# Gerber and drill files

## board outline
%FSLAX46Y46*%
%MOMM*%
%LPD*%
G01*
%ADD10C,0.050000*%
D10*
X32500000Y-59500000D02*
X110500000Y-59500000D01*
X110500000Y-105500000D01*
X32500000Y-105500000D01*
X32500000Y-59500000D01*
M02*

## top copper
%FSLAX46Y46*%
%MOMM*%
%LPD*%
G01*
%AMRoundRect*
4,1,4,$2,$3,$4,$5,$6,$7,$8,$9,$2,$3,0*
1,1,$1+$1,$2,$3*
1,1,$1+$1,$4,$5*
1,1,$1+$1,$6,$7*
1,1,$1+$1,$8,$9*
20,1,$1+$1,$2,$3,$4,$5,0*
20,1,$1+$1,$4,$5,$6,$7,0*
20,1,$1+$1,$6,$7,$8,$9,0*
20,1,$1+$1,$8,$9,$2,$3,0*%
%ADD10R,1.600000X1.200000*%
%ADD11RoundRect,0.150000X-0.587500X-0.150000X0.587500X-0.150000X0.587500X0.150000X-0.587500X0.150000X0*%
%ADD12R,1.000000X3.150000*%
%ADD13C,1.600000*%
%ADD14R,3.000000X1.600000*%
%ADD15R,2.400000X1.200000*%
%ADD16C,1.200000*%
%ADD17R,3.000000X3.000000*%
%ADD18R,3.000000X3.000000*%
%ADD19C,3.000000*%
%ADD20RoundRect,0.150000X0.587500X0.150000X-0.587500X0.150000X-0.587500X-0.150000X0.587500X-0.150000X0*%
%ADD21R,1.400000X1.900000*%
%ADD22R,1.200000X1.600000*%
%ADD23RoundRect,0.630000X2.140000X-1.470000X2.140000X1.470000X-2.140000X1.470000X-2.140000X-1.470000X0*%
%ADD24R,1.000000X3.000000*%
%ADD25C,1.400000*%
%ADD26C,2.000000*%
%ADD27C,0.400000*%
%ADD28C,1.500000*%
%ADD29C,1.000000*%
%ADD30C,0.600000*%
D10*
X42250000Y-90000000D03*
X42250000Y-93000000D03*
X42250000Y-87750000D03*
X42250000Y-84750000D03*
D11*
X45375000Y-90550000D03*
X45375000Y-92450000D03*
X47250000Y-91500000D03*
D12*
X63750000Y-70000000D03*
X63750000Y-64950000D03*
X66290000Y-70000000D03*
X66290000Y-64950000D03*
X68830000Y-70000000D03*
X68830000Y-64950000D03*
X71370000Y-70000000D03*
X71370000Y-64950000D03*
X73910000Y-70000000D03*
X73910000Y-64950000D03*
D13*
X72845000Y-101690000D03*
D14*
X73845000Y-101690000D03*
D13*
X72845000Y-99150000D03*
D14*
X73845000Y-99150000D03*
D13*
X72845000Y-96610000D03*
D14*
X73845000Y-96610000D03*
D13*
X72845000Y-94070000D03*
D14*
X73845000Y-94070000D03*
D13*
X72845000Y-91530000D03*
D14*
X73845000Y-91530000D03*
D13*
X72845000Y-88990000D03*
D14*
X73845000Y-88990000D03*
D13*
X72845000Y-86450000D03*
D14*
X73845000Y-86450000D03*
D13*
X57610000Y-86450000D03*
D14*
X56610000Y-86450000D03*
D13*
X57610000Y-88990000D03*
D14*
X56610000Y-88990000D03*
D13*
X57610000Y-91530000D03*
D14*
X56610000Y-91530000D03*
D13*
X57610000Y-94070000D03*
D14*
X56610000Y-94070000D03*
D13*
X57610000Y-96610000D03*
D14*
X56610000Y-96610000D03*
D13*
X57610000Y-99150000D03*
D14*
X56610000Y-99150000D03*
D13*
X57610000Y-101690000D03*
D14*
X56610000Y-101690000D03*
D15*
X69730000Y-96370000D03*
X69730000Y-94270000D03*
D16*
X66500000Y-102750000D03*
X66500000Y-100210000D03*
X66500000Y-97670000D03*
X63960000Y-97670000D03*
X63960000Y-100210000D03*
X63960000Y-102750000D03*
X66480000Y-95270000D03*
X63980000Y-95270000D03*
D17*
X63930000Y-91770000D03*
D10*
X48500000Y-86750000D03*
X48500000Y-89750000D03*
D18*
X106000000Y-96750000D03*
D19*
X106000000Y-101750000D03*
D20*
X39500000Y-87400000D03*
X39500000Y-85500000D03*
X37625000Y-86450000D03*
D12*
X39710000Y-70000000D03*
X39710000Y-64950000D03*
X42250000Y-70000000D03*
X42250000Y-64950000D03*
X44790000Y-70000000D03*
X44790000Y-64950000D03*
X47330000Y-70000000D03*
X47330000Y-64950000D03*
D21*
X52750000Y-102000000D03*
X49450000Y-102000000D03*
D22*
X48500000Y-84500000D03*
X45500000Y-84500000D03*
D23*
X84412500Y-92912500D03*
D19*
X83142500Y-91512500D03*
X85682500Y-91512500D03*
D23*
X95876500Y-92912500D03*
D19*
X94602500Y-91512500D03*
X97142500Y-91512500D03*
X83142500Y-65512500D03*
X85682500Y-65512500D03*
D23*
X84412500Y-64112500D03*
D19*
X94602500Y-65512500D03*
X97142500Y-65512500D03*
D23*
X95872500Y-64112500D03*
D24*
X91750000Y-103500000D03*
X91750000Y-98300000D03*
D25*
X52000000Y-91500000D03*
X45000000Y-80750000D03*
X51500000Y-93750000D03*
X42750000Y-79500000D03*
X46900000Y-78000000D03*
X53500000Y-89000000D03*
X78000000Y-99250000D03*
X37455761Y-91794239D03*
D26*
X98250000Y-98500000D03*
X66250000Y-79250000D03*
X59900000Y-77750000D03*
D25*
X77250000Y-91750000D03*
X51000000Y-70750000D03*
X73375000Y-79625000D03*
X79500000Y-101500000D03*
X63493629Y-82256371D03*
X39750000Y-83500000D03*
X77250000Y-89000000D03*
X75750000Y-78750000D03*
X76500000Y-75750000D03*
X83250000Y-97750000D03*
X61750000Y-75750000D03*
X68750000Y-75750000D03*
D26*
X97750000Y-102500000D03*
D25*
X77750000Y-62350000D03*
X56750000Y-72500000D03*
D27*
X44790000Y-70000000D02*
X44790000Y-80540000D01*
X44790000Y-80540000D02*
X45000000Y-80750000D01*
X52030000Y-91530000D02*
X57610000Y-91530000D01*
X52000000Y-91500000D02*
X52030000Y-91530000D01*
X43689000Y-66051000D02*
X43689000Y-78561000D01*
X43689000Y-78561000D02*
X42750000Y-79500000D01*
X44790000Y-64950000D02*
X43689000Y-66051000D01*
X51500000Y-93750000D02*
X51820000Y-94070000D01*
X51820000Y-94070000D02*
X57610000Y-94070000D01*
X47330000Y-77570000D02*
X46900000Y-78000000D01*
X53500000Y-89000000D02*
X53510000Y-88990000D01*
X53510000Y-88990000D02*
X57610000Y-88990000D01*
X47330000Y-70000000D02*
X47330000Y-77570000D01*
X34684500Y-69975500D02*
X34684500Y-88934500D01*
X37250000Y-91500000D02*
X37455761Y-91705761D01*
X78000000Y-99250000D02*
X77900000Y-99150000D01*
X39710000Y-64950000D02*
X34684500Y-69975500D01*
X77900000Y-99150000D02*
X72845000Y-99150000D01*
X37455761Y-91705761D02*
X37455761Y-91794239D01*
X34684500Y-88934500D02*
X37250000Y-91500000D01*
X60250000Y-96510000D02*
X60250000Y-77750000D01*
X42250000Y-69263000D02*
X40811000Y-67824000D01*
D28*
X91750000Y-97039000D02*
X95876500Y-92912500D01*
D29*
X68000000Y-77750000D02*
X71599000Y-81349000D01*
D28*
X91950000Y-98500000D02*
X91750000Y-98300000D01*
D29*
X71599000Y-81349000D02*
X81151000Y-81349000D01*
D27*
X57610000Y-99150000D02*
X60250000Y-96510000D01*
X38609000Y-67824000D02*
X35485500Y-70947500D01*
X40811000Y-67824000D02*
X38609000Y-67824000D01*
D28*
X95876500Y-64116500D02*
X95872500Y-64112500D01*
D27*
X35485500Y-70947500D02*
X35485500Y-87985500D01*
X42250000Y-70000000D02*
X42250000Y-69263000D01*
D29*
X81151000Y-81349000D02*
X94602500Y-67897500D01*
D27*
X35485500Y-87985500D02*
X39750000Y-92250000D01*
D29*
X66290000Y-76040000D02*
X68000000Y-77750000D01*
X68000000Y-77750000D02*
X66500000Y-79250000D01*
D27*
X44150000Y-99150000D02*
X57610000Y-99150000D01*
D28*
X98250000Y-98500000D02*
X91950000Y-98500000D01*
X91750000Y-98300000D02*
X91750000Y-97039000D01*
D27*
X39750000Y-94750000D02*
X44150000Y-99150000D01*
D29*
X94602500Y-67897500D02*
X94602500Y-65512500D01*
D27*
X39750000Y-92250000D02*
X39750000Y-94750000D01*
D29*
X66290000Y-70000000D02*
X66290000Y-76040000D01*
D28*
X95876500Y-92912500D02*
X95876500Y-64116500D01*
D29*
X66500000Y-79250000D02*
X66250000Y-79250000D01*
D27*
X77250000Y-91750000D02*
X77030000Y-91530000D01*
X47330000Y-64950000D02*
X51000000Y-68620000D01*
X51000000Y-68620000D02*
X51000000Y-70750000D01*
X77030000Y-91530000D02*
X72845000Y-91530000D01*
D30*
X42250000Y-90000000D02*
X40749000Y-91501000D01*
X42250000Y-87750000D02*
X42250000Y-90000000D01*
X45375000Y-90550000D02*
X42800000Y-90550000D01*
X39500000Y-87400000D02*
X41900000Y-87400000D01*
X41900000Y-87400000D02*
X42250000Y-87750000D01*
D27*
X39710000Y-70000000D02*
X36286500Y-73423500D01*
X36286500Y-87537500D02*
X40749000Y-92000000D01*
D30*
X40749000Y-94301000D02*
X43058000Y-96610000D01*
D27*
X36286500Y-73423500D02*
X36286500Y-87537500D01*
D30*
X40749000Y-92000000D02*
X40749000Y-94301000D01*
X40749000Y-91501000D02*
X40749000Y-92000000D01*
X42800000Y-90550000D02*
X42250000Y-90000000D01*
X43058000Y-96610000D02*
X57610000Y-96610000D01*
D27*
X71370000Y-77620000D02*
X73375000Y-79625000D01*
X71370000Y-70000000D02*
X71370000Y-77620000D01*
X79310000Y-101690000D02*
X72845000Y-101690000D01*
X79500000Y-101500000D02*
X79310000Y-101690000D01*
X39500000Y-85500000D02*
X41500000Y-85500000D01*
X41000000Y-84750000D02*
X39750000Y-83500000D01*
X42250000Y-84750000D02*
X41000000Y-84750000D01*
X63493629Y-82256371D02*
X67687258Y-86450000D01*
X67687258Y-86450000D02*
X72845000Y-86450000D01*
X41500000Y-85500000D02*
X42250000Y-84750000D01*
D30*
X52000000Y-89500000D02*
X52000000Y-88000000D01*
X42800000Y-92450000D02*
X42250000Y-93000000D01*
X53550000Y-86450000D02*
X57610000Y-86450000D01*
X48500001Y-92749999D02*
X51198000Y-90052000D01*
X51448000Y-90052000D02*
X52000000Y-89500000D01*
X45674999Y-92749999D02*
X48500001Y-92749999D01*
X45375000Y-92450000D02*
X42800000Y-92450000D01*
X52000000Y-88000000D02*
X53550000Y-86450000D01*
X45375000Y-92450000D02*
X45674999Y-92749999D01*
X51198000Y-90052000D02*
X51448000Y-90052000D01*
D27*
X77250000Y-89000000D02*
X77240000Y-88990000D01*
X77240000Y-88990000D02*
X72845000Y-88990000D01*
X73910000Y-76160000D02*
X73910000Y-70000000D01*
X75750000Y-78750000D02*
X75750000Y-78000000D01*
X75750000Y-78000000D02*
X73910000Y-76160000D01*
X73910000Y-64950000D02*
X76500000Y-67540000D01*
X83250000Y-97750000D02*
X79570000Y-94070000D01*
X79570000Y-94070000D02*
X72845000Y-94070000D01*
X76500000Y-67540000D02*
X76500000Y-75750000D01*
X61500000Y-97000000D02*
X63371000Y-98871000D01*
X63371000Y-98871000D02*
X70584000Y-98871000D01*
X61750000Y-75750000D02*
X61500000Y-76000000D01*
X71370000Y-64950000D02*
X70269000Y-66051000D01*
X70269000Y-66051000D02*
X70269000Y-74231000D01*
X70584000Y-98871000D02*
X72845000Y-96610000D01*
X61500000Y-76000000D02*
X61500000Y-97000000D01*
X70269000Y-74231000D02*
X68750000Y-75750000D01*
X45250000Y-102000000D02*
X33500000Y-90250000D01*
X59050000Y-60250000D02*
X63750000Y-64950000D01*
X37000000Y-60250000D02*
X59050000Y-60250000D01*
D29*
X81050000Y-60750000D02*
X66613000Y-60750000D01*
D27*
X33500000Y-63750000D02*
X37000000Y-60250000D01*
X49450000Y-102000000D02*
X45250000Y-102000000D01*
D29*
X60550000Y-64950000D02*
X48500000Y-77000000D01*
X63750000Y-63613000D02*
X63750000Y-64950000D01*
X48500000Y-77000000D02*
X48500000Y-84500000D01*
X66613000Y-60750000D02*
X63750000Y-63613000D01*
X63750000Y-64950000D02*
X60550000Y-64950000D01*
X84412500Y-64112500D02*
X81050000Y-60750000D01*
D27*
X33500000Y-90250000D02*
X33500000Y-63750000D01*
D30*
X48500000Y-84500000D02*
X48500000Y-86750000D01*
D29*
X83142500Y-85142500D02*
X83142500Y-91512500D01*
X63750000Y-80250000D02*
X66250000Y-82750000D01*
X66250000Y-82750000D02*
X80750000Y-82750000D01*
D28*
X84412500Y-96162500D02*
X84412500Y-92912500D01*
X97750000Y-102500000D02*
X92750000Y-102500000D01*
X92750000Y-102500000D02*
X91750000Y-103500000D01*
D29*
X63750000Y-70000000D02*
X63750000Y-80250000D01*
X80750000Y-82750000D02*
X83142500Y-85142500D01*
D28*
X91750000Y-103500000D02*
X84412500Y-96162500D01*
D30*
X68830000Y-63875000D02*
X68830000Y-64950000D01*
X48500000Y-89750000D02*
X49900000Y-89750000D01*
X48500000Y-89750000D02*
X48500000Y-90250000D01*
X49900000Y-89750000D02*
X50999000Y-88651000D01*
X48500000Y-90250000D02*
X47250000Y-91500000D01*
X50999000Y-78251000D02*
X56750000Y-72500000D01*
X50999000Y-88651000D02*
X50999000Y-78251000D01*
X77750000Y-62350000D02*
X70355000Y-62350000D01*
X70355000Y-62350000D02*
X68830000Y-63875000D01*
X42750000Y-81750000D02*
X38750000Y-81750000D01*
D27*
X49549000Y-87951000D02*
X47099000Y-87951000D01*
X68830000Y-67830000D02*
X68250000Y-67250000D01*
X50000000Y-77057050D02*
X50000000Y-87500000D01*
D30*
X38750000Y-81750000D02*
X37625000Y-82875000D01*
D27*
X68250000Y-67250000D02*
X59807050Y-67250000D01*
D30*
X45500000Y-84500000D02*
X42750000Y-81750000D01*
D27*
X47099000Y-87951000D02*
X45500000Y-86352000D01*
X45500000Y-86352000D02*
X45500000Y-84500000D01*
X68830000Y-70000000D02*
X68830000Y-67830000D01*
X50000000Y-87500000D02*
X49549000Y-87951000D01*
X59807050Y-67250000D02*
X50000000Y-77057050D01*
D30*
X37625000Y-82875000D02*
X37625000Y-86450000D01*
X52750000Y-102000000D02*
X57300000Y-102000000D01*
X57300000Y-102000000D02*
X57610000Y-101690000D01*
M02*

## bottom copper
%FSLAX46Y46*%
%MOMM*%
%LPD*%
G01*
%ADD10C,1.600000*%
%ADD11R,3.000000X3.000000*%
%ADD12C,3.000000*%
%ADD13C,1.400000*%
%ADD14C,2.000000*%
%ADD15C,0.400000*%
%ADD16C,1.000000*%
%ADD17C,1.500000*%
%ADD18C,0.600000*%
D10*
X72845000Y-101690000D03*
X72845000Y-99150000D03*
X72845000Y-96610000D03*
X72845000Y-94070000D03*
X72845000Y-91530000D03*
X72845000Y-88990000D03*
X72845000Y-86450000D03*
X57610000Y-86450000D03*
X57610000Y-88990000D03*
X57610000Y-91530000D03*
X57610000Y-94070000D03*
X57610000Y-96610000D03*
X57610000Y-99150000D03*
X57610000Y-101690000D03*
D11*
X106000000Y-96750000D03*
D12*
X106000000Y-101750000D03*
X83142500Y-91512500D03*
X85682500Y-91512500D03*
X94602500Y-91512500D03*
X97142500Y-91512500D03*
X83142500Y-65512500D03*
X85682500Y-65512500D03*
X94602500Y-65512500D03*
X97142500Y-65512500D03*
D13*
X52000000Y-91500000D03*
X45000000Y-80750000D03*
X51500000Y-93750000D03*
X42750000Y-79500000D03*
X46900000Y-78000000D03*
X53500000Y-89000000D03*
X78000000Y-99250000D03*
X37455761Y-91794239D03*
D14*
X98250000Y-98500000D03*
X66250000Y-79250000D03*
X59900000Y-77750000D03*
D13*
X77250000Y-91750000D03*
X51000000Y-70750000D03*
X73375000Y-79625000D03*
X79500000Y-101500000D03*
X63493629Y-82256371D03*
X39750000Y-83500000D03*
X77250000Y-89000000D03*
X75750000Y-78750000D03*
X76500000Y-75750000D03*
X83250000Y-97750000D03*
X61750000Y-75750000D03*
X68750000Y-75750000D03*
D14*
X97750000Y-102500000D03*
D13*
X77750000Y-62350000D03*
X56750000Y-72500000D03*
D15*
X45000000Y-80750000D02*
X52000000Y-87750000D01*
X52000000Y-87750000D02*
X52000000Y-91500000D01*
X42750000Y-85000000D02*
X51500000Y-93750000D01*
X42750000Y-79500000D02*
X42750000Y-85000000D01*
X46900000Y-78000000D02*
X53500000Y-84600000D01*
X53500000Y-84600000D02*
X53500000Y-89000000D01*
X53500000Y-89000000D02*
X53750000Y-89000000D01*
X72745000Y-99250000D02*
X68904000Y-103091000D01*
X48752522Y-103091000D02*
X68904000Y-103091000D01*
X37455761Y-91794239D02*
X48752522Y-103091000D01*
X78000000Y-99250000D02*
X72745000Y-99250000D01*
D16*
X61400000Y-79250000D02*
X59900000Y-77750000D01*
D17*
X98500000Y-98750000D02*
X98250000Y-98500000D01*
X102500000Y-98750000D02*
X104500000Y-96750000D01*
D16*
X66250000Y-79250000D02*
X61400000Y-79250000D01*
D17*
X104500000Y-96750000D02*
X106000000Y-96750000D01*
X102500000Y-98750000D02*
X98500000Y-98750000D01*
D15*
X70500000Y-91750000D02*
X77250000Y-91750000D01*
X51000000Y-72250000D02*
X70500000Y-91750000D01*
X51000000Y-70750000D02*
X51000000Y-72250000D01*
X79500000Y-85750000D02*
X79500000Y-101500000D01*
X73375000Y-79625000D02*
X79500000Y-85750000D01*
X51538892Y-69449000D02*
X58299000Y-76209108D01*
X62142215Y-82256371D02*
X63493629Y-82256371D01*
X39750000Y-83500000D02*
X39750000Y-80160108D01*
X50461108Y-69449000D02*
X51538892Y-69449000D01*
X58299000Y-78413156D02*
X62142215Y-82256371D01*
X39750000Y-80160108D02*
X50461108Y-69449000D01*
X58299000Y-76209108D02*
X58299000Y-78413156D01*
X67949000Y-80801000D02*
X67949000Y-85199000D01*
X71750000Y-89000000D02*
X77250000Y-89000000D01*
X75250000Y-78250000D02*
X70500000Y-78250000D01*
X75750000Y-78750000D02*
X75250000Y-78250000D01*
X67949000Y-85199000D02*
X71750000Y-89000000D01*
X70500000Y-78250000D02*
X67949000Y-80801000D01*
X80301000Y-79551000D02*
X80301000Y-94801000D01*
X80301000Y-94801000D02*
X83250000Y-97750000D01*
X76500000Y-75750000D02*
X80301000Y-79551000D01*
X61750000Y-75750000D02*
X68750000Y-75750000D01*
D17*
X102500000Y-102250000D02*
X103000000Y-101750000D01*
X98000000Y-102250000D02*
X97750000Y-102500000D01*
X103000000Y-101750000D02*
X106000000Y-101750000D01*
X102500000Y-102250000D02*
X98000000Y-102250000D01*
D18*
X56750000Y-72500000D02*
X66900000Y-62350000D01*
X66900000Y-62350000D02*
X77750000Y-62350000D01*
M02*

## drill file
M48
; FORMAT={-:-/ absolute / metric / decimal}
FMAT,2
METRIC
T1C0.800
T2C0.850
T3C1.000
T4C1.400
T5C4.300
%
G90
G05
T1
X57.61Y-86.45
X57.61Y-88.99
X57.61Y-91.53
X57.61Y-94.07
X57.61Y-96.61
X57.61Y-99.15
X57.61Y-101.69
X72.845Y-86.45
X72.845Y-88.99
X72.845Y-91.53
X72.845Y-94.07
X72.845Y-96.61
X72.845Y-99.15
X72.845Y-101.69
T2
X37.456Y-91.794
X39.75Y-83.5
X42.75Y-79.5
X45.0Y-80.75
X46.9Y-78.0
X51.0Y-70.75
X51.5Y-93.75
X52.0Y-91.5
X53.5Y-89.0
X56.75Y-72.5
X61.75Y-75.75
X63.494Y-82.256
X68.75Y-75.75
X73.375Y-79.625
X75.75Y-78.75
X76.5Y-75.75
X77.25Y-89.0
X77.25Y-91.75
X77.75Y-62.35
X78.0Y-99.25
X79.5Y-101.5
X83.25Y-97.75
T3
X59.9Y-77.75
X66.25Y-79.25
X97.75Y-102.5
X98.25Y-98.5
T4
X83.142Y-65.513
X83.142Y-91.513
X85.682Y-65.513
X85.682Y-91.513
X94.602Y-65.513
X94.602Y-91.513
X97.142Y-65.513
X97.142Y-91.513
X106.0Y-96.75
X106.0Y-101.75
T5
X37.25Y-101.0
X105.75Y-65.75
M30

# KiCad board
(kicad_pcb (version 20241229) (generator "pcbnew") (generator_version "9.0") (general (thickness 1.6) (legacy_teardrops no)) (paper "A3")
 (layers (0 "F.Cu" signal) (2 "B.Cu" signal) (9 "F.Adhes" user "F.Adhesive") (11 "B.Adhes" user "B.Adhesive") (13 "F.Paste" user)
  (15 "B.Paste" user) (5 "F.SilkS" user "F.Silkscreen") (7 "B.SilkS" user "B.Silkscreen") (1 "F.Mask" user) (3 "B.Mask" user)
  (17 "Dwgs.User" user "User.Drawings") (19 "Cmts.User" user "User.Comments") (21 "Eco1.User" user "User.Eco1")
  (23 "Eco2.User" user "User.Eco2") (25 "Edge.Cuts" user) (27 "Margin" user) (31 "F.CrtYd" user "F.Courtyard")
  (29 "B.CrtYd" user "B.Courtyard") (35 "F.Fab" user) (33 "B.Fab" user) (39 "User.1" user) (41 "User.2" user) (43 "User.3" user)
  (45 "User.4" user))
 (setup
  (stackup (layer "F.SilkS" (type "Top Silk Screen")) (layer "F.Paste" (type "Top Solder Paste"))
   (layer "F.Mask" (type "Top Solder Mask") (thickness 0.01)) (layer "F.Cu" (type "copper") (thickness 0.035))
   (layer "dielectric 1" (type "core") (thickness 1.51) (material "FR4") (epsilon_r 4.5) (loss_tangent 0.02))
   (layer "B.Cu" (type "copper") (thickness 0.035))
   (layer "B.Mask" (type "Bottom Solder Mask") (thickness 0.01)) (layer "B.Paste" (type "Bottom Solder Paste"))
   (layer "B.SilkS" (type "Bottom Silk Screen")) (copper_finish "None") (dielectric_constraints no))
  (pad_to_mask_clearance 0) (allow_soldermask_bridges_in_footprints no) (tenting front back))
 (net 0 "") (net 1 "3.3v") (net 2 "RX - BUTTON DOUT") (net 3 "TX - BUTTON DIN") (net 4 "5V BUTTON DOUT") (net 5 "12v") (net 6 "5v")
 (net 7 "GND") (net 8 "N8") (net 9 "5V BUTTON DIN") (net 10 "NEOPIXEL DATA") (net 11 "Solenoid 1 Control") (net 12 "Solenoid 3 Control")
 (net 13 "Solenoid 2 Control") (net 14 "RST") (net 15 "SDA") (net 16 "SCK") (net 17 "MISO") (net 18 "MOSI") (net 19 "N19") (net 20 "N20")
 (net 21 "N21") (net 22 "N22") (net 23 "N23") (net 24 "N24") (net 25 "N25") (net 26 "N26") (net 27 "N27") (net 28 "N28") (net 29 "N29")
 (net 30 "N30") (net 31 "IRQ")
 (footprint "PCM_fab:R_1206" (layer "F.Cu") (at 42.25 91.5 -90)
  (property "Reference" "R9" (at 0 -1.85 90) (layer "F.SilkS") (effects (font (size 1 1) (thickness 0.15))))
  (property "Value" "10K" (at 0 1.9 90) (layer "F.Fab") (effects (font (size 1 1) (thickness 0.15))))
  (pad "1" smd rect (at -1.5 0 270) (size 1.2 1.6) (layers "F.Cu" "F.Mask" "F.Paste") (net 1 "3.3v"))
  (pad "2" smd rect (at 1.5 0 270) (size 1.2 1.6) (layers "F.Cu" "F.Mask" "F.Paste") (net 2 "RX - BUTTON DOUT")))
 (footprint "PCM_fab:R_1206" (layer "F.Cu") (at 42.25 86.25 90)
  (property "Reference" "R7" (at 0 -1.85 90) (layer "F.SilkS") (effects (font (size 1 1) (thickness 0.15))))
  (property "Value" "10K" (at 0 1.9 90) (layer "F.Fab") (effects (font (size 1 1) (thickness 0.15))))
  (pad "1" smd rect (at -1.5 0 90) (size 1.2 1.6) (layers "F.Cu" "F.Mask" "F.Paste") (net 1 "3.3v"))
  (pad "2" smd rect (at 1.5 0 90) (size 1.2 1.6) (layers "F.Cu" "F.Mask" "F.Paste") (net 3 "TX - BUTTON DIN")))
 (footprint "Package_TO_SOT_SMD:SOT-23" (layer "F.Cu") (at 46.3125 91.5)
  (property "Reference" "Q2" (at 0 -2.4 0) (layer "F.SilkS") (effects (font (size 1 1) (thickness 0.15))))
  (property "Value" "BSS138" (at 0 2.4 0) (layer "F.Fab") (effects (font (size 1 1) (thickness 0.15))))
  (pad "1" smd roundrect (at -0.9375 -0.95) (size 1.475 0.6) (layers "F.Cu" "F.Mask" "F.Paste") (roundrect_rratio 0.25) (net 1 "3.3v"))
  (pad "2" smd roundrect (at -0.9375 0.95) (size 1.475 0.6) (layers "F.Cu" "F.Mask" "F.Paste") (roundrect_rratio 0.25)
   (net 2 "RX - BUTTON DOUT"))
  (pad "3" smd roundrect (at 0.9375 0) (size 1.475 0.6) (layers "F.Cu" "F.Mask" "F.Paste") (roundrect_rratio 0.25) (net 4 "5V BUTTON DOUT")))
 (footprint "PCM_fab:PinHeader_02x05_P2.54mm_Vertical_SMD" (layer "F.Cu") (at 68.83 67.475 90)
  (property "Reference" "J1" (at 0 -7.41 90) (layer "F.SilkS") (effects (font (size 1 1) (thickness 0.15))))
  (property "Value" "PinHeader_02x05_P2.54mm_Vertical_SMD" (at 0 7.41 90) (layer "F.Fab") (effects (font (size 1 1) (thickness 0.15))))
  (pad "1" smd rect (at -2.525 -5.08 90) (size 3.15 1) (layers "F.Cu" "F.Mask" "F.Paste") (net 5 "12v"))
  (pad "2" smd rect (at 2.525 -5.08 90) (size 3.15 1) (layers "F.Cu" "F.Mask" "F.Paste") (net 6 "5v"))
  (pad "3" smd rect (at -2.525 -2.54 90) (size 3.15 1) (layers "F.Cu" "F.Mask" "F.Paste") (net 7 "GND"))
  (pad "4" smd rect (at 2.525 -2.54 90) (size 3.15 1) (layers "F.Cu" "F.Mask" "F.Paste") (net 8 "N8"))
  (pad "5" smd rect (at -2.525 0 90) (size 3.15 1) (layers "F.Cu" "F.Mask" "F.Paste") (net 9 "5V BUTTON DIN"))
  (pad "6" smd rect (at 2.525 0 90) (size 3.15 1) (layers "F.Cu" "F.Mask" "F.Paste") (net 4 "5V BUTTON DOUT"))
  (pad "7" smd rect (at -2.525 2.54 90) (size 3.15 1) (layers "F.Cu" "F.Mask" "F.Paste") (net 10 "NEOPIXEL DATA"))
  (pad "8" smd rect (at 2.525 2.54 90) (size 3.15 1) (layers "F.Cu" "F.Mask" "F.Paste") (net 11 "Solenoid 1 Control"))
  (pad "9" smd rect (at -2.525 5.08 90) (size 3.15 1) (layers "F.Cu" "F.Mask" "F.Paste") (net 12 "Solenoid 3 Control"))
  (pad "10" smd rect (at 2.525 5.08 90) (size 3.15 1) (layers "F.Cu" "F.Mask" "F.Paste") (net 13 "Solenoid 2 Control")))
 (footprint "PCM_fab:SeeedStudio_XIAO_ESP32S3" (layer "F.Cu") (at 65.23 94.07 180)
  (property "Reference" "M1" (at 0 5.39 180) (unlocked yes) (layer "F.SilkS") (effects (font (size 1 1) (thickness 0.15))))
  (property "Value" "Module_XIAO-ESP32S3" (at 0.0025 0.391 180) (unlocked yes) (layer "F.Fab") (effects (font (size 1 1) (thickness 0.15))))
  (pad "1" thru_hole circle (at -7.615 -7.62 180) (size 1.6 1.6) (drill 0.8) (layers "*.Cu" "*.Mask") (remove_unused_layers no)
   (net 10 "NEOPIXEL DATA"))
  (pad "1" smd rect (at -7.615 -7.62 180) (size 3 1.6) (drill (offset -1 0)) (layers "F.Cu" "F.Mask" "F.Paste") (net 10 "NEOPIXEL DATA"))
  (pad "2" thru_hole circle (at -7.615 -5.08 180) (size 1.6 1.6) (drill 0.8) (layers "*.Cu" "*.Mask") (remove_unused_layers no)
   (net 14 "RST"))
  (pad "2" smd rect (at -7.615 -5.08 180) (size 3 1.6) (drill (offset -1 0)) (layers "F.Cu" "F.Mask" "F.Paste") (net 14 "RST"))
  (pad "3" thru_hole circle (at -7.615 -2.54 180) (size 1.6 1.6) (drill 0.8) (layers "*.Cu" "*.Mask") (remove_unused_layers no)
   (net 11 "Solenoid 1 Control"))
  (pad "3" smd rect (at -7.615 -2.54 180) (size 3 1.6) (drill (offset -1 0)) (layers "F.Cu" "F.Mask" "F.Paste")
   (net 11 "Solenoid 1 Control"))
  (pad "4" thru_hole circle (at -7.615 0 180) (size 1.6 1.6) (drill 0.8) (layers "*.Cu" "*.Mask") (remove_unused_layers no)
   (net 13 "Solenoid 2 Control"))
  (pad "4" smd rect (at -7.615 0 180) (size 3 1.6) (drill (offset -1 0)) (layers "F.Cu" "F.Mask" "F.Paste") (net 13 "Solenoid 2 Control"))
  (pad "5" thru_hole circle (at -7.615 2.54 180) (size 1.6 1.6) (drill 0.8) (layers "*.Cu" "*.Mask") (remove_unused_layers no)
   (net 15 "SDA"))
  (pad "5" smd rect (at -7.615 2.54 180) (size 3 1.6) (drill (offset -1 0)) (layers "F.Cu" "F.Mask" "F.Paste") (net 15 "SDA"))
  (pad "6" thru_hole circle (at -7.615 5.08 180) (size 1.6 1.6) (drill 0.8) (layers "*.Cu" "*.Mask") (remove_unused_layers no)
   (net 12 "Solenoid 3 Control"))
  (pad "6" smd rect (at -7.615 5.08 180) (size 3 1.6) (drill (offset -1 0)) (layers "F.Cu" "F.Mask" "F.Paste") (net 12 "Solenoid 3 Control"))
  (pad "7" thru_hole circle (at -7.615 7.62 180) (size 1.6 1.6) (drill 0.8) (layers "*.Cu" "*.Mask") (remove_unused_layers no)
   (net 3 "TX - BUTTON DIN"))
  (pad "7" smd rect (at -7.615 7.62 180) (size 3 1.6) (drill (offset -1 0)) (layers "F.Cu" "F.Mask" "F.Paste") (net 3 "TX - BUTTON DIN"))
  (pad "8" thru_hole circle (at 7.62 7.62 180) (size 1.6 1.6) (drill 0.8) (layers "*.Cu" "*.Mask") (remove_unused_layers no)
   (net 2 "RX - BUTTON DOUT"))
  (pad "8" smd rect (at 7.62 7.62 180) (size 3 1.6) (drill (offset 1 0)) (layers "F.Cu" "F.Mask" "F.Paste") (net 2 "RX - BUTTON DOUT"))
  (pad "9" thru_hole circle (at 7.62 5.08 180) (size 1.6 1.6) (drill 0.8) (layers "*.Cu" "*.Mask") (remove_unused_layers no) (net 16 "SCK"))
  (pad "9" smd rect (at 7.62 5.08 180) (size 3 1.6) (drill (offset 1 0)) (layers "F.Cu" "F.Mask" "F.Paste") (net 16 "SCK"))
  (pad "10" thru_hole circle (at 7.62 2.54 180) (size 1.6 1.6) (drill 0.8) (layers "*.Cu" "*.Mask") (remove_unused_layers no)
   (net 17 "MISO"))
  (pad "10" smd rect (at 7.62 2.54 180) (size 3 1.6) (drill (offset 1 0)) (layers "F.Cu" "F.Mask" "F.Paste") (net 17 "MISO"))
  (pad "11" thru_hole circle (at 7.62 0 180) (size 1.6 1.6) (drill 0.8) (layers "*.Cu" "*.Mask") (remove_unused_layers no) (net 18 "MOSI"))
  (pad "11" smd rect (at 7.62 0 180) (size 3 1.6) (drill (offset 1 0)) (layers "F.Cu" "F.Mask" "F.Paste") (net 18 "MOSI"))
  (pad "12" thru_hole circle (at 7.62 -2.54 180) (size 1.6 1.6) (drill 0.8) (layers "*.Cu" "*.Mask") (remove_unused_layers no)
   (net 1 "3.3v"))
  (pad "12" smd rect (at 7.62 -2.54 180) (size 3 1.6) (drill (offset 1 0)) (layers "F.Cu" "F.Mask" "F.Paste") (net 1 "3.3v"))
  (pad "13" thru_hole circle (at 7.62 -5.08 180) (size 1.6 1.6) (drill 0.8) (layers "*.Cu" "*.Mask") (remove_unused_layers no) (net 7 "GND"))
  (pad "13" smd rect (at 7.62 -5.08 180) (size 3 1.6) (drill (offset 1 0)) (layers "F.Cu" "F.Mask" "F.Paste") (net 7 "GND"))
  (pad "14" thru_hole circle (at 7.62 -7.62 180) (size 1.6 1.6) (drill 0.8) (layers "*.Cu" "*.Mask") (remove_unused_layers no)
   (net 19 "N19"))
  (pad "14" smd rect (at 7.62 -7.62 180) (size 3 1.6) (drill (offset 1 0)) (layers "F.Cu" "F.Mask" "F.Paste") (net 19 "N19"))
  (pad "15" smd rect (at -4.5 -2.3 180) (size 2.4 1.2) (layers "F.Cu" "F.Mask" "F.Paste") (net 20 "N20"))
  (pad "16" smd rect (at -4.5 -0.2 180) (size 2.4 1.2) (layers "F.Cu" "F.Mask" "F.Paste") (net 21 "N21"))
  (pad "17" smd circle (at -1.27 -8.68 180) (size 1.2 1.2) (layers "F.Cu" "F.Mask" "F.Paste") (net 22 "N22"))
  (pad "18" smd circle (at -1.27 -6.14 180) (size 1.2 1.2) (layers "F.Cu" "F.Mask" "F.Paste") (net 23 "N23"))
  (pad "19" smd circle (at -1.27 -3.6 180) (size 1.2 1.2) (layers "F.Cu" "F.Mask" "F.Paste") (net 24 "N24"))
  (pad "20" smd circle (at 1.27 -3.6 180) (size 1.2 1.2) (layers "F.Cu" "F.Mask" "F.Paste") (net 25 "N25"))
  (pad "21" smd circle (at 1.27 -6.14 180) (size 1.2 1.2) (layers "F.Cu" "F.Mask" "F.Paste") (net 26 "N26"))
  (pad "22" smd circle (at 1.27 -8.68 180) (size 1.2 1.2) (layers "F.Cu" "F.Mask" "F.Paste") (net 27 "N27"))
  (pad "23" smd circle (at -1.25 -1.2 180) (size 1.2 1.2) (layers "F.Cu" "F.Mask" "F.Paste") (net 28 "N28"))
  (pad "24" smd circle (at 1.25 -1.2 180) (size 1.2 1.2) (layers "F.Cu" "F.Mask" "F.Paste") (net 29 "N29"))
  (pad "25" smd rect (at 1.3 2.3 180) (size 3 3) (layers "F.Cu" "F.Mask" "F.Paste") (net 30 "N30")))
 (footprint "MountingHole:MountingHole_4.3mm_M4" (layer "F.Cu") (at 105.75 65.75)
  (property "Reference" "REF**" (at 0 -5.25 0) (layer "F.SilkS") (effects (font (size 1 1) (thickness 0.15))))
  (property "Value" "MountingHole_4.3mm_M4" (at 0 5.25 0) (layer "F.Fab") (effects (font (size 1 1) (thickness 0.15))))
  (pad "" np_thru_hole circle (at 0 0) (size 4.3 4.3) (drill 4.3) (layers "*.Cu" "*.Mask")))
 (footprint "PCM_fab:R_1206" (layer "F.Cu") (at 48.5 88.25 -90)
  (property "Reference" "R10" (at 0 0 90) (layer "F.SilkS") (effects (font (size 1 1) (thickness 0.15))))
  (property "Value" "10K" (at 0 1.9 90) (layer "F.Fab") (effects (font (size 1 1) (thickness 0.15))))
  (pad "1" smd rect (at -1.5 0 270) (size 1.2 1.6) (layers "F.Cu" "F.Mask" "F.Paste") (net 6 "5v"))
  (pad "2" smd rect (at 1.5 0 270) (size 1.2 1.6) (layers "F.Cu" "F.Mask" "F.Paste") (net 4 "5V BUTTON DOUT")))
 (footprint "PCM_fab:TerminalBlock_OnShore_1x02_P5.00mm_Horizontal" (layer "F.Cu") (at 106 96.75 -90)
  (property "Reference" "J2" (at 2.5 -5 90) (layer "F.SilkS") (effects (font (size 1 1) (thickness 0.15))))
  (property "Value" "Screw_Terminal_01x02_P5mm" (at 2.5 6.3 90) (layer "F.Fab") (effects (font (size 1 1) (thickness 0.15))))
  (pad "1" thru_hole rect (at 0 0 270) (size 3 3) (drill 1.4) (layers "*.Cu" "*.Mask") (remove_unused_layers no) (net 7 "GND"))
  (pad "2" thru_hole circle (at 5 0 270) (size 3 3) (drill 1.4) (layers "*.Cu" "*.Mask") (remove_unused_layers no) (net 5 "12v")))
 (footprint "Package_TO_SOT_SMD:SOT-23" (layer "F.Cu") (at 38.5625 86.45 180)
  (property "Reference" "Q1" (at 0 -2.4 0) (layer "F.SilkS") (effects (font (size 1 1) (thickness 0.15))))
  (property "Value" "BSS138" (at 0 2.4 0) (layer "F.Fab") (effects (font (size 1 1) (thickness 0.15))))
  (pad "1" smd roundrect (at -0.9375 -0.95 180) (size 1.475 0.6) (layers "F.Cu" "F.Mask" "F.Paste") (roundrect_rratio 0.25) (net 1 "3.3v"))
  (pad "2" smd roundrect (at -0.9375 0.95 180) (size 1.475 0.6) (layers "F.Cu" "F.Mask" "F.Paste") (roundrect_rratio 0.25)
   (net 3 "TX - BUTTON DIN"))
  (pad "3" smd roundrect (at 0.9375 0 180) (size 1.475 0.6) (layers "F.Cu" "F.Mask" "F.Paste") (roundrect_rratio 0.25)
   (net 9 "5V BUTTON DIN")))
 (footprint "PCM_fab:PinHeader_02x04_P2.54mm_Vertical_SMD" (layer "F.Cu") (at 43.52 67.475 90)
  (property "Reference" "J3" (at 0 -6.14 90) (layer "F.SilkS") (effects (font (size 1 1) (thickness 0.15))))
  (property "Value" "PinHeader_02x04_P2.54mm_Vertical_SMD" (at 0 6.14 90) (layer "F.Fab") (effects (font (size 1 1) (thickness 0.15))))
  (pad "1" smd rect (at -2.525 -3.81 90) (size 3.15 1) (layers "F.Cu" "F.Mask" "F.Paste") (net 1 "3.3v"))
  (pad "2" smd rect (at 2.525 -3.81 90) (size 3.15 1) (layers "F.Cu" "F.Mask" "F.Paste") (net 14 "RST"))
  (pad "3" smd rect (at -2.525 -1.27 90) (size 3.15 1) (layers "F.Cu" "F.Mask" "F.Paste") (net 7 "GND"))
  (pad "4" smd rect (at 2.525 -1.27 90) (size 3.15 1) (layers "F.Cu" "F.Mask" "F.Paste") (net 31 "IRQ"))
  (pad "5" smd rect (at -2.525 1.27 90) (size 3.15 1) (layers "F.Cu" "F.Mask" "F.Paste") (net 17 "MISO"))
  (pad "6" smd rect (at 2.525 1.27 90) (size 3.15 1) (layers "F.Cu" "F.Mask" "F.Paste") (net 18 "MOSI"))
  (pad "7" smd rect (at -2.525 3.81 90) (size 3.15 1) (layers "F.Cu" "F.Mask" "F.Paste") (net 16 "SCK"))
  (pad "8" smd rect (at 2.525 3.81 90) (size 3.15 1) (layers "F.Cu" "F.Mask" "F.Paste") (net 15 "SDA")))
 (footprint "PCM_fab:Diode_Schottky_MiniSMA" (layer "F.Cu") (at 51.1 102 180)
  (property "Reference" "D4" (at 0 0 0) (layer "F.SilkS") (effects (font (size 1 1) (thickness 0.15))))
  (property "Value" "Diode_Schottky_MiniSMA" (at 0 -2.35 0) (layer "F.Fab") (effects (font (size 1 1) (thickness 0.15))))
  (pad "1" smd rect (at -1.65 0 180) (size 1.4 1.9) (layers "F.Cu" "F.Mask" "F.Paste") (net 19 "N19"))
  (pad "2" smd rect (at 1.65 0 180) (size 1.4 1.9) (layers "F.Cu" "F.Mask" "F.Paste") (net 6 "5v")))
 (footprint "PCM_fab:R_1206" (layer "F.Cu") (at 47 84.5 180)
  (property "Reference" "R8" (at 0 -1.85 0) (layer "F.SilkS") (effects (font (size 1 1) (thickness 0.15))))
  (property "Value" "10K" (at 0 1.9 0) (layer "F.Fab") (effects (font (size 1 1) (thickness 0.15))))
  (pad "1" smd rect (at -1.5 0 180) (size 1.2 1.6) (layers "F.Cu" "F.Mask" "F.Paste") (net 6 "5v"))
  (pad "2" smd rect (at 1.5 0 180) (size 1.2 1.6) (layers "F.Cu" "F.Mask" "F.Paste") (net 9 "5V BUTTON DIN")))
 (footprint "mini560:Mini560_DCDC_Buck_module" (layer "F.Cu") (at 90.1425 78.5125 90)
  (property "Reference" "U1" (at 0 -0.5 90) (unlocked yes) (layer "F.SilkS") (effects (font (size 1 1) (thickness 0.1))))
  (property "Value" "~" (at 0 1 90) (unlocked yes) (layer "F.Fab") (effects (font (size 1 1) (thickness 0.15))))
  (pad "1" smd roundrect (at -14.4 -5.73 90) (size 4.2 5.54) (layers "F.Cu" "F.Mask" "F.Paste") (roundrect_rratio 0.15) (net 5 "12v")
   (thermal_bridge_angle 45))
  (pad "1" thru_hole circle (at -13 -7 90) (size 3 3) (drill 1.4) (layers "*.Cu" "*.Mask") (remove_unused_layers no) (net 5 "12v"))
  (pad "1" thru_hole circle (at -13 -4.46 90) (size 3 3) (drill 1.4) (layers "*.Cu" "*.Mask") (remove_unused_layers no) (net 5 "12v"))
  (pad "2" smd roundrect (at -14.4 5.734 90) (size 4.2 5.54) (layers "F.Cu" "F.Mask" "F.Paste") (roundrect_rratio 0.15) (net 7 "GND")
   (thermal_bridge_angle 45))
  (pad "2" thru_hole circle (at -13 4.46 90) (size 3 3) (drill 1.4) (layers "*.Cu" "*.Mask") (remove_unused_layers no) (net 7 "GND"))
  (pad "2" thru_hole circle (at -13 7 90) (size 3 3) (drill 1.4) (layers "*.Cu" "*.Mask") (remove_unused_layers no) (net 7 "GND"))
  (pad "3" thru_hole circle (at 13 -7 90) (size 3 3) (drill 1.4) (layers "*.Cu" "*.Mask") (remove_unused_layers no) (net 6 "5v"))
  (pad "3" thru_hole circle (at 13 -4.46 90) (size 3 3) (drill 1.4) (layers "*.Cu" "*.Mask") (remove_unused_layers no) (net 6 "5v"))
  (pad "3" smd roundrect (at 14.4 -5.73 90) (size 4.2 5.54) (layers "F.Cu" "F.Mask" "F.Paste") (roundrect_rratio 0.15) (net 6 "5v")
   (thermal_bridge_angle 45))
  (pad "4" thru_hole circle (at 13 4.46 90) (size 3 3) (drill 1.4) (layers "*.Cu" "*.Mask") (remove_unused_layers no) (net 7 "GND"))
  (pad "4" thru_hole circle (at 13 7 90) (size 3 3) (drill 1.4) (layers "*.Cu" "*.Mask") (remove_unused_layers no) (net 7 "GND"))
  (pad "4" smd roundrect (at 14.4 5.73 90) (size 4.2 5.54) (layers "F.Cu" "F.Mask" "F.Paste") (roundrect_rratio 0.15) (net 7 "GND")
   (thermal_bridge_angle 45)))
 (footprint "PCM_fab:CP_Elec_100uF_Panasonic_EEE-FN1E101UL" (layer "F.Cu") (at 91.75 100.9 90)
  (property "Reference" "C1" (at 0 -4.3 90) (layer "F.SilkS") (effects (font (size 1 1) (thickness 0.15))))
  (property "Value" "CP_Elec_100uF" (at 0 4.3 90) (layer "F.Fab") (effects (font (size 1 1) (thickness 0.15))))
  (pad "1" smd rect (at -2.6 0 90) (size 3 1) (layers "F.Cu" "F.Mask" "F.Paste") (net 5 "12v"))
  (pad "2" smd rect (at 2.6 0 90) (size 3 1) (layers "F.Cu" "F.Mask" "F.Paste") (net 7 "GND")))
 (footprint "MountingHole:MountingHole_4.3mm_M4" (layer "F.Cu") (at 37.25 101)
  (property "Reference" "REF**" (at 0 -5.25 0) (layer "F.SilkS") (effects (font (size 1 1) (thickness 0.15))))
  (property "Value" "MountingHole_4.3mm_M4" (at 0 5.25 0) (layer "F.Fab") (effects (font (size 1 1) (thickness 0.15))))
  (pad "" np_thru_hole circle (at 0 0) (size 4.3 4.3) (drill 4.3) (layers "*.Cu" "*.Mask")))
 (gr_rect (start 32.5 59.5) (end 110.5 105.5) (stroke (width 0.05) (type default)) (fill no) (layer "Edge.Cuts"))
 (segment (start 44.79 70) (end 44.79 80.54) (width 0.4) (layer "F.Cu") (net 17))
 (segment (start 44.79 80.54) (end 45 80.75) (width 0.4) (layer "F.Cu") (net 17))
 (segment (start 52.03 91.53) (end 57.61 91.53) (width 0.4) (layer "F.Cu") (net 17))
 (segment (start 52 91.5) (end 52.03 91.53) (width 0.4) (layer "F.Cu") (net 17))
 (via (at 52 91.5) (size 1.4) (drill 0.85) (layers "F.Cu" "B.Cu") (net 17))
 (via (at 45 80.75) (size 1.4) (drill 0.85) (layers "F.Cu" "B.Cu") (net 17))
 (segment (start 45 80.75) (end 52 87.75) (width 0.4) (layer "B.Cu") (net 17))
 (segment (start 52 87.75) (end 52 91.5) (width 0.4) (layer "B.Cu") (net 17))
 (segment (start 43.689 66.051) (end 43.689 78.561) (width 0.4) (layer "F.Cu") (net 18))
 (segment (start 43.689 78.561) (end 42.75 79.5) (width 0.4) (layer "F.Cu") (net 18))
 (segment (start 44.79 64.95) (end 43.689 66.051) (width 0.4) (layer "F.Cu") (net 18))
 (segment (start 51.5 93.75) (end 51.82 94.07) (width 0.4) (layer "F.Cu") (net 18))
 (segment (start 51.82 94.07) (end 57.61 94.07) (width 0.4) (layer "F.Cu") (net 18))
 (via (at 51.5 93.75) (size 1.4) (drill 0.85) (layers "F.Cu" "B.Cu") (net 18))
 (via (at 42.75 79.5) (size 1.4) (drill 0.85) (layers "F.Cu" "B.Cu") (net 18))
 (segment (start 42.75 85) (end 51.5 93.75) (width 0.4) (layer "B.Cu") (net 18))
 (segment (start 42.75 79.5) (end 42.75 85) (width 0.4) (layer "B.Cu") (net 18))
 (segment (start 47.33 77.57) (end 46.9 78) (width 0.4) (layer "F.Cu") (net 16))
 (segment (start 53.5 89) (end 53.51 88.99) (width 0.4) (layer "F.Cu") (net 16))
 (segment (start 53.51 88.99) (end 57.61 88.99) (width 0.4) (layer "F.Cu") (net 16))
 (segment (start 47.33 70) (end 47.33 77.57) (width 0.4) (layer "F.Cu") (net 16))
 (via (at 46.9 78) (size 1.4) (drill 0.85) (layers "F.Cu" "B.Cu") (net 16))
 (via (at 53.5 89) (size 1.4) (drill 0.85) (layers "F.Cu" "B.Cu") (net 16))
 (segment (start 46.9 78) (end 53.5 84.6) (width 0.4) (layer "B.Cu") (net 16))
 (segment (start 53.5 84.6) (end 53.5 89) (width 0.4) (layer "B.Cu") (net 16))
 (segment (start 53.5 89) (end 53.75 89) (width 0.4) (layer "B.Cu") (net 16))
 (segment (start 34.6845 69.9755) (end 34.6845 88.9345) (width 0.4) (layer "F.Cu") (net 14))
 (segment (start 37.25 91.5) (end 37.455761 91.705761) (width 0.4) (layer "F.Cu") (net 14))
 (segment (start 78 99.25) (end 77.9 99.15) (width 0.4) (layer "F.Cu") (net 14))
 (segment (start 39.71 64.95) (end 34.6845 69.9755) (width 0.4) (layer "F.Cu") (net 14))
 (segment (start 77.9 99.15) (end 72.845 99.15) (width 0.4) (layer "F.Cu") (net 14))
 (segment (start 37.455761 91.705761) (end 37.455761 91.794239) (width 0.4) (layer "F.Cu") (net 14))
 (segment (start 34.6845 88.9345) (end 37.25 91.5) (width 0.4) (layer "F.Cu") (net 14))
 (via (at 78 99.25) (size 1.4) (drill 0.85) (layers "F.Cu" "B.Cu") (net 14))
 (via (at 37.455761 91.794239) (size 1.4) (drill 0.85) (layers "F.Cu" "B.Cu") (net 14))
 (segment (start 72.745 99.25) (end 68.904 103.091) (width 0.4) (layer "B.Cu") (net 14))
 (segment (start 48.752522 103.091) (end 68.904 103.091) (width 0.4) (layer "B.Cu") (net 14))
 (segment (start 37.455761 91.794239) (end 48.752522 103.091) (width 0.4) (layer "B.Cu") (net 14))
 (segment (start 78 99.25) (end 72.745 99.25) (width 0.4) (layer "B.Cu") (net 14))
 (segment (start 60.25 96.51) (end 60.25 77.75) (width 0.4) (layer "F.Cu") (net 7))
 (segment (start 42.25 69.263) (end 40.811 67.824) (width 0.4) (layer "F.Cu") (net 7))
 (segment (start 91.75 97.039) (end 95.8765 92.9125) (width 1.5) (layer "F.Cu") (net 7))
 (segment (start 68 77.75) (end 71.599 81.349) (width 1) (layer "F.Cu") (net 7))
 (segment (start 91.95 98.5) (end 91.75 98.3) (width 1.5) (layer "F.Cu") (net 7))
 (segment (start 71.599 81.349) (end 81.151 81.349) (width 1) (layer "F.Cu") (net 7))
 (segment (start 57.61 99.15) (end 60.25 96.51) (width 0.4) (layer "F.Cu") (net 7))
 (segment (start 38.609 67.824) (end 35.4855 70.9475) (width 0.4) (layer "F.Cu") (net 7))
 (segment (start 40.811 67.824) (end 38.609 67.824) (width 0.4) (layer "F.Cu") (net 7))
 (segment (start 95.8765 64.1165) (end 95.8725 64.1125) (width 1.5) (layer "F.Cu") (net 7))
 (segment (start 35.4855 70.9475) (end 35.4855 87.9855) (width 0.4) (layer "F.Cu") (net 7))
 (segment (start 42.25 70) (end 42.25 69.263) (width 0.4) (layer "F.Cu") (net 7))
 (segment (start 81.151 81.349) (end 94.6025 67.8975) (width 1) (layer "F.Cu") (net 7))
 (segment (start 35.4855 87.9855) (end 39.75 92.25) (width 0.4) (layer "F.Cu") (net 7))
 (segment (start 66.29 76.04) (end 68 77.75) (width 1) (layer "F.Cu") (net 7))
 (segment (start 68 77.75) (end 66.5 79.25) (width 1) (layer "F.Cu") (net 7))
 (segment (start 44.15 99.15) (end 57.61 99.15) (width 0.4) (layer "F.Cu") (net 7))
 (segment (start 98.25 98.5) (end 91.95 98.5) (width 1.5) (layer "F.Cu") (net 7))
 (segment (start 91.75 98.3) (end 91.75 97.039) (width 1.5) (layer "F.Cu") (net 7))
 (segment (start 39.75 94.75) (end 44.15 99.15) (width 0.4) (layer "F.Cu") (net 7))
 (segment (start 94.6025 67.8975) (end 94.6025 65.5125) (width 1) (layer "F.Cu") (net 7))
 (segment (start 39.75 92.25) (end 39.75 94.75) (width 0.4) (layer "F.Cu") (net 7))
 (segment (start 66.29 70) (end 66.29 76.04) (width 1) (layer "F.Cu") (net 7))
 (segment (start 95.8765 92.9125) (end 95.8765 64.1165) (width 1.5) (layer "F.Cu") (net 7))
 (segment (start 66.5 79.25) (end 66.25 79.25) (width 1) (layer "F.Cu") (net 7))
 (via (at 98.25 98.5) (size 2) (drill 1) (layers "F.Cu" "B.Cu") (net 7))
 (via (at 66.25 79.25) (size 2) (drill 1) (layers "F.Cu" "B.Cu") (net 7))
 (via (at 59.9 77.75) (size 2) (drill 1) (layers "F.Cu" "B.Cu") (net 7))
 (segment (start 61.4 79.25) (end 59.9 77.75) (width 1) (layer "B.Cu") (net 7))
 (segment (start 98.5 98.75) (end 98.25 98.5) (width 1.5) (layer "B.Cu") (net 7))
 (segment (start 102.5 98.75) (end 104.5 96.75) (width 1.5) (layer "B.Cu") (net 7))
 (segment (start 66.25 79.25) (end 61.4 79.25) (width 1) (layer "B.Cu") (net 7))
 (segment (start 104.5 96.75) (end 106 96.75) (width 1.5) (layer "B.Cu") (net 7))
 (segment (start 102.5 98.75) (end 98.5 98.75) (width 1.5) (layer "B.Cu") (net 7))
 (segment (start 77.25 91.75) (end 77.03 91.53) (width 0.4) (layer "F.Cu") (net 15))
 (segment (start 47.33 64.95) (end 51 68.62) (width 0.4) (layer "F.Cu") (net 15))
 (segment (start 51 68.62) (end 51 70.75) (width 0.4) (layer "F.Cu") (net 15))
 (segment (start 77.03 91.53) (end 72.845 91.53) (width 0.4) (layer "F.Cu") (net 15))
 (via (at 77.25 91.75) (size 1.4) (drill 0.85) (layers "F.Cu" "B.Cu") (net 15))
 (via (at 51 70.75) (size 1.4) (drill 0.85) (layers "F.Cu" "B.Cu") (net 15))
 (segment (start 70.5 91.75) (end 77.25 91.75) (width 0.4) (layer "B.Cu") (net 15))
 (segment (start 51 72.25) (end 70.5 91.75) (width 0.4) (layer "B.Cu") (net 15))
 (segment (start 51 70.75) (end 51 72.25) (width 0.4) (layer "B.Cu") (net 15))
 (segment (start 42.25 90) (end 40.749 91.501) (width 0.6) (layer "F.Cu") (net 1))
 (segment (start 42.25 87.75) (end 42.25 90) (width 0.6) (layer "F.Cu") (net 1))
 (segment (start 45.375 90.55) (end 42.8 90.55) (width 0.6) (layer "F.Cu") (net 1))
 (segment (start 39.5 87.4) (end 41.9 87.4) (width 0.6) (layer "F.Cu") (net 1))
 (segment (start 41.9 87.4) (end 42.25 87.75) (width 0.6) (layer "F.Cu") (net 1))
 (segment (start 39.71 70) (end 36.2865 73.4235) (width 0.4) (layer "F.Cu") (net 1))
 (segment (start 36.2865 87.5375) (end 40.749 92) (width 0.4) (layer "F.Cu") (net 1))
 (segment (start 40.749 94.301) (end 43.058 96.61) (width 0.6) (layer "F.Cu") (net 1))
 (segment (start 36.2865 73.4235) (end 36.2865 87.5375) (width 0.4) (layer "F.Cu") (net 1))
 (segment (start 40.749 92) (end 40.749 94.301) (width 0.6) (layer "F.Cu") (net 1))
 (segment (start 40.749 91.501) (end 40.749 92) (width 0.6) (layer "F.Cu") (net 1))
 (segment (start 42.8 90.55) (end 42.25 90) (width 0.6) (layer "F.Cu") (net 1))
 (segment (start 43.058 96.61) (end 57.61 96.61) (width 0.6) (layer "F.Cu") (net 1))
 (segment (start 71.37 77.62) (end 73.375 79.625) (width 0.4) (layer "F.Cu") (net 10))
 (segment (start 71.37 70) (end 71.37 77.62) (width 0.4) (layer "F.Cu") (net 10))
 (segment (start 79.31 101.69) (end 72.845 101.69) (width 0.4) (layer "F.Cu") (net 10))
 (segment (start 79.5 101.5) (end 79.31 101.69) (width 0.4) (layer "F.Cu") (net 10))
 (via (at 73.375 79.625) (size 1.4) (drill 0.85) (layers "F.Cu" "B.Cu") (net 10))
 (via (at 79.5 101.5) (size 1.4) (drill 0.85) (layers "F.Cu" "B.Cu") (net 10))
 (segment (start 79.5 85.75) (end 79.5 101.5) (width 0.4) (layer "B.Cu") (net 10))
 (segment (start 73.375 79.625) (end 79.5 85.75) (width 0.4) (layer "B.Cu") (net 10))
 (segment (start 39.5 85.5) (end 41.5 85.5) (width 0.4) (layer "F.Cu") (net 3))
 (segment (start 41 84.75) (end 39.75 83.5) (width 0.4) (layer "F.Cu") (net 3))
 (segment (start 42.25 84.75) (end 41 84.75) (width 0.4) (layer "F.Cu") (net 3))
 (segment (start 63.493629 82.256371) (end 67.687258 86.45) (width 0.4) (layer "F.Cu") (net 3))
 (segment (start 67.687258 86.45) (end 72.845 86.45) (width 0.4) (layer "F.Cu") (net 3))
 (segment (start 41.5 85.5) (end 42.25 84.75) (width 0.4) (layer "F.Cu") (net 3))
 (via (at 63.493629 82.256371) (size 1.4) (drill 0.85) (layers "F.Cu" "B.Cu") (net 3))
 (via (at 39.75 83.5) (size 1.4) (drill 0.85) (layers "F.Cu" "B.Cu") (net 3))
 (segment (start 51.538892 69.449) (end 58.299 76.209108) (width 0.4) (layer "B.Cu") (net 3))
 (segment (start 62.142215 82.256371) (end 63.493629 82.256371) (width 0.4) (layer "B.Cu") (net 3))
 (segment (start 39.75 83.5) (end 39.75 80.160108) (width 0.4) (layer "B.Cu") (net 3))
 (segment (start 50.461108 69.449) (end 51.538892 69.449) (width 0.4) (layer "B.Cu") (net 3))
 (segment (start 58.299 78.413156) (end 62.142215 82.256371) (width 0.4) (layer "B.Cu") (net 3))
 (segment (start 39.75 80.160108) (end 50.461108 69.449) (width 0.4) (layer "B.Cu") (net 3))
 (segment (start 58.299 76.209108) (end 58.299 78.413156) (width 0.4) (layer "B.Cu") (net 3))
 (segment (start 52 89.5) (end 52 88) (width 0.6) (layer "F.Cu") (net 2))
 (segment (start 42.8 92.45) (end 42.25 93) (width 0.6) (layer "F.Cu") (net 2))
 (segment (start 53.55 86.45) (end 57.61 86.45) (width 0.6) (layer "F.Cu") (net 2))
 (segment (start 48.500001 92.749999) (end 51.198 90.052) (width 0.6) (layer "F.Cu") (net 2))
 (segment (start 51.448 90.052) (end 52 89.5) (width 0.6) (layer "F.Cu") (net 2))
 (segment (start 45.674999 92.749999) (end 48.500001 92.749999) (width 0.6) (layer "F.Cu") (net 2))
 (segment (start 45.375 92.45) (end 42.8 92.45) (width 0.6) (layer "F.Cu") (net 2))
 (segment (start 52 88) (end 53.55 86.45) (width 0.6) (layer "F.Cu") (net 2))
 (segment (start 45.375 92.45) (end 45.674999 92.749999) (width 0.6) (layer "F.Cu") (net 2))
 (segment (start 51.198 90.052) (end 51.448 90.052) (width 0.6) (layer "F.Cu") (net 2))
 (segment (start 77.25 89) (end 77.24 88.99) (width 0.4) (layer "F.Cu") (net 12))
 (segment (start 77.24 88.99) (end 72.845 88.99) (width 0.4) (layer "F.Cu") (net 12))
 (segment (start 73.91 76.16) (end 73.91 70) (width 0.4) (layer "F.Cu") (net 12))
 (segment (start 75.75 78.75) (end 75.75 78) (width 0.4) (layer "F.Cu") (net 12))
 (segment (start 75.75 78) (end 73.91 76.16) (width 0.4) (layer "F.Cu") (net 12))
 (via (at 77.25 89) (size 1.4) (drill 0.85) (layers "F.Cu" "B.Cu") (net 12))
 (via (at 75.75 78.75) (size 1.4) (drill 0.85) (layers "F.Cu" "B.Cu") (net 12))
 (segment (start 67.949 80.801) (end 67.949 85.199) (width 0.4) (layer "B.Cu") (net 12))
 (segment (start 71.75 89) (end 77.25 89) (width 0.4) (layer "B.Cu") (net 12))
 (segment (start 75.25 78.25) (end 70.5 78.25) (width 0.4) (layer "B.Cu") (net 12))
 (segment (start 75.75 78.75) (end 75.25 78.25) (width 0.4) (layer "B.Cu") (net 12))
 (segment (start 67.949 85.199) (end 71.75 89) (width 0.4) (layer "B.Cu") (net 12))
 (segment (start 70.5 78.25) (end 67.949 80.801) (width 0.4) (layer "B.Cu") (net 12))
 (segment (start 73.91 64.95) (end 76.5 67.54) (width 0.4) (layer "F.Cu") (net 13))
 (segment (start 83.25 97.75) (end 79.57 94.07) (width 0.4) (layer "F.Cu") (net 13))
 (segment (start 79.57 94.07) (end 72.845 94.07) (width 0.4) (layer "F.Cu") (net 13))
 (segment (start 76.5 67.54) (end 76.5 75.75) (width 0.4) (layer "F.Cu") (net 13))
 (via (at 76.5 75.75) (size 1.4) (drill 0.85) (layers "F.Cu" "B.Cu") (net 13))
 (via (at 83.25 97.75) (size 1.4) (drill 0.85) (layers "F.Cu" "B.Cu") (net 13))
 (segment (start 80.301 79.551) (end 80.301 94.801) (width 0.4) (layer "B.Cu") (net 13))
 (segment (start 80.301 94.801) (end 83.25 97.75) (width 0.4) (layer "B.Cu") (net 13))
 (segment (start 76.5 75.75) (end 80.301 79.551) (width 0.4) (layer "B.Cu") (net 13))
 (segment (start 61.5 97) (end 63.371 98.871) (width 0.4) (layer "F.Cu") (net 11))
 (segment (start 63.371 98.871) (end 70.584 98.871) (width 0.4) (layer "F.Cu") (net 11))
 (segment (start 61.75 75.75) (end 61.5 76) (width 0.4) (layer "F.Cu") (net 11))
 (segment (start 71.37 64.95) (end 70.269 66.051) (width 0.4) (layer "F.Cu") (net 11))
 (segment (start 70.269 66.051) (end 70.269 74.231) (width 0.4) (layer "F.Cu") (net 11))
 (segment (start 70.584 98.871) (end 72.845 96.61) (width 0.4) (layer "F.Cu") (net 11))
 (segment (start 61.5 76) (end 61.5 97) (width 0.4) (layer "F.Cu") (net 11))
 (segment (start 70.269 74.231) (end 68.75 75.75) (width 0.4) (layer "F.Cu") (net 11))
 (via (at 61.75 75.75) (size 1.4) (drill 0.85) (layers "F.Cu" "B.Cu") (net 11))
 (via (at 68.75 75.75) (size 1.4) (drill 0.85) (layers "F.Cu" "B.Cu") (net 11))
 (segment (start 61.75 75.75) (end 68.75 75.75) (width 0.4) (layer "B.Cu") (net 11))
 (segment (start 45.25 102) (end 33.5 90.25) (width 0.4) (layer "F.Cu") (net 6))
 (segment (start 59.05 60.25) (end 63.75 64.95) (width 0.4) (layer "F.Cu") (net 6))
 (segment (start 37 60.25) (end 59.05 60.25) (width 0.4) (layer "F.Cu") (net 6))
 (segment (start 81.05 60.75) (end 66.613 60.75) (width 1) (layer "F.Cu") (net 6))
 (segment (start 33.5 63.75) (end 37 60.25) (width 0.4) (layer "F.Cu") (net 6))
 (segment (start 49.45 102) (end 45.25 102) (width 0.4) (layer "F.Cu") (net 6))
 (segment (start 60.55 64.95) (end 48.5 77) (width 1) (layer "F.Cu") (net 6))
 (segment (start 63.75 63.613) (end 63.75 64.95) (width 1) (layer "F.Cu") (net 6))
 (segment (start 48.5 77) (end 48.5 84.5) (width 1) (layer "F.Cu") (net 6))
 (segment (start 66.613 60.75) (end 63.75 63.613) (width 1) (layer "F.Cu") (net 6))
 (segment (start 63.75 64.95) (end 60.55 64.95) (width 1) (layer "F.Cu") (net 6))
 (segment (start 84.4125 64.1125) (end 81.05 60.75) (width 1) (layer "F.Cu") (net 6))
 (segment (start 33.5 90.25) (end 33.5 63.75) (width 0.4) (layer "F.Cu") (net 6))
 (segment (start 48.5 84.5) (end 48.5 86.75) (width 0.6) (layer "F.Cu") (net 6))
 (segment (start 83.1425 85.1425) (end 83.1425 91.5125) (width 1) (layer "F.Cu") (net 5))
 (segment (start 63.75 80.25) (end 66.25 82.75) (width 1) (layer "F.Cu") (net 5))
 (segment (start 66.25 82.75) (end 80.75 82.75) (width 1) (layer "F.Cu") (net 5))
 (segment (start 84.4125 96.1625) (end 84.4125 92.9125) (width 1.5) (layer "F.Cu") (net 5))
 (segment (start 97.75 102.5) (end 92.75 102.5) (width 1.5) (layer "F.Cu") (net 5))
 (segment (start 92.75 102.5) (end 91.75 103.5) (width 1.5) (layer "F.Cu") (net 5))
 (segment (start 63.75 70) (end 63.75 80.25) (width 1) (layer "F.Cu") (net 5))
 (segment (start 80.75 82.75) (end 83.1425 85.1425) (width 1) (layer "F.Cu") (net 5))
 (segment (start 91.75 103.5) (end 84.4125 96.1625) (width 1.5) (layer "F.Cu") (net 5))
 (via (at 97.75 102.5) (size 2) (drill 1) (layers "F.Cu" "B.Cu") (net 5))
 (segment (start 102.5 102.25) (end 103 101.75) (width 1.5) (layer "B.Cu") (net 5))
 (segment (start 98 102.25) (end 97.75 102.5) (width 1.5) (layer "B.Cu") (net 5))
 (segment (start 103 101.75) (end 106 101.75) (width 1.5) (layer "B.Cu") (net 5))
 (segment (start 102.5 102.25) (end 98 102.25) (width 1.5) (layer "B.Cu") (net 5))
 (segment (start 68.83 63.875) (end 68.83 64.95) (width 0.6) (layer "F.Cu") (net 4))
 (segment (start 48.5 89.75) (end 49.9 89.75) (width 0.6) (layer "F.Cu") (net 4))
 (segment (start 48.5 89.75) (end 48.5 90.25) (width 0.6) (layer "F.Cu") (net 4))
 (segment (start 49.9 89.75) (end 50.999 88.651) (width 0.6) (layer "F.Cu") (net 4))
 (segment (start 48.5 90.25) (end 47.25 91.5) (width 0.6) (layer "F.Cu") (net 4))
 (segment (start 50.999 78.251) (end 56.75 72.5) (width 0.6) (layer "F.Cu") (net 4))
 (segment (start 50.999 88.651) (end 50.999 78.251) (width 0.6) (layer "F.Cu") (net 4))
 (segment (start 77.75 62.35) (end 70.355 62.35) (width 0.6) (layer "F.Cu") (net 4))
 (segment (start 70.355 62.35) (end 68.83 63.875) (width 0.6) (layer "F.Cu") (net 4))
 (via (at 77.75 62.35) (size 1.4) (drill 0.85) (layers "F.Cu" "B.Cu") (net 4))
 (via (at 56.75 72.5) (size 1.4) (drill 0.85) (layers "F.Cu" "B.Cu") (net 4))
 (segment (start 56.75 72.5) (end 66.9 62.35) (width 0.6) (layer "B.Cu") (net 4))
 (segment (start 66.9 62.35) (end 77.75 62.35) (width 0.6) (layer "B.Cu") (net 4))
 (segment (start 42.75 81.75) (end 38.75 81.75) (width 0.6) (layer "F.Cu") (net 9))
 (segment (start 49.549 87.951) (end 47.099 87.951) (width 0.4) (layer "F.Cu") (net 9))
 (segment (start 68.83 67.83) (end 68.25 67.25) (width 0.4) (layer "F.Cu") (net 9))
 (segment (start 50 77.05705) (end 50 87.5) (width 0.4) (layer "F.Cu") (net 9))
 (segment (start 38.75 81.75) (end 37.625 82.875) (width 0.6) (layer "F.Cu") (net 9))
 (segment (start 68.25 67.25) (end 59.80705 67.25) (width 0.4) (layer "F.Cu") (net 9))
 (segment (start 45.5 84.5) (end 42.75 81.75) (width 0.6) (layer "F.Cu") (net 9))
 (segment (start 47.099 87.951) (end 45.5 86.352) (width 0.4) (layer "F.Cu") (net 9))
 (segment (start 45.5 86.352) (end 45.5 84.5) (width 0.4) (layer "F.Cu") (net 9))
 (segment (start 68.83 70) (end 68.83 67.83) (width 0.4) (layer "F.Cu") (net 9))
 (segment (start 50 87.5) (end 49.549 87.951) (width 0.4) (layer "F.Cu") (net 9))
 (segment (start 59.80705 67.25) (end 50 77.05705) (width 0.4) (layer "F.Cu") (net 9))
 (segment (start 37.625 82.875) (end 37.625 86.45) (width 0.6) (layer "F.Cu") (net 9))
 (segment (start 52.75 102) (end 57.3 102) (width 0.6) (layer "F.Cu") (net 19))
 (segment (start 57.3 102) (end 57.61 101.69) (width 0.6) (layer "F.Cu") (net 19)))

